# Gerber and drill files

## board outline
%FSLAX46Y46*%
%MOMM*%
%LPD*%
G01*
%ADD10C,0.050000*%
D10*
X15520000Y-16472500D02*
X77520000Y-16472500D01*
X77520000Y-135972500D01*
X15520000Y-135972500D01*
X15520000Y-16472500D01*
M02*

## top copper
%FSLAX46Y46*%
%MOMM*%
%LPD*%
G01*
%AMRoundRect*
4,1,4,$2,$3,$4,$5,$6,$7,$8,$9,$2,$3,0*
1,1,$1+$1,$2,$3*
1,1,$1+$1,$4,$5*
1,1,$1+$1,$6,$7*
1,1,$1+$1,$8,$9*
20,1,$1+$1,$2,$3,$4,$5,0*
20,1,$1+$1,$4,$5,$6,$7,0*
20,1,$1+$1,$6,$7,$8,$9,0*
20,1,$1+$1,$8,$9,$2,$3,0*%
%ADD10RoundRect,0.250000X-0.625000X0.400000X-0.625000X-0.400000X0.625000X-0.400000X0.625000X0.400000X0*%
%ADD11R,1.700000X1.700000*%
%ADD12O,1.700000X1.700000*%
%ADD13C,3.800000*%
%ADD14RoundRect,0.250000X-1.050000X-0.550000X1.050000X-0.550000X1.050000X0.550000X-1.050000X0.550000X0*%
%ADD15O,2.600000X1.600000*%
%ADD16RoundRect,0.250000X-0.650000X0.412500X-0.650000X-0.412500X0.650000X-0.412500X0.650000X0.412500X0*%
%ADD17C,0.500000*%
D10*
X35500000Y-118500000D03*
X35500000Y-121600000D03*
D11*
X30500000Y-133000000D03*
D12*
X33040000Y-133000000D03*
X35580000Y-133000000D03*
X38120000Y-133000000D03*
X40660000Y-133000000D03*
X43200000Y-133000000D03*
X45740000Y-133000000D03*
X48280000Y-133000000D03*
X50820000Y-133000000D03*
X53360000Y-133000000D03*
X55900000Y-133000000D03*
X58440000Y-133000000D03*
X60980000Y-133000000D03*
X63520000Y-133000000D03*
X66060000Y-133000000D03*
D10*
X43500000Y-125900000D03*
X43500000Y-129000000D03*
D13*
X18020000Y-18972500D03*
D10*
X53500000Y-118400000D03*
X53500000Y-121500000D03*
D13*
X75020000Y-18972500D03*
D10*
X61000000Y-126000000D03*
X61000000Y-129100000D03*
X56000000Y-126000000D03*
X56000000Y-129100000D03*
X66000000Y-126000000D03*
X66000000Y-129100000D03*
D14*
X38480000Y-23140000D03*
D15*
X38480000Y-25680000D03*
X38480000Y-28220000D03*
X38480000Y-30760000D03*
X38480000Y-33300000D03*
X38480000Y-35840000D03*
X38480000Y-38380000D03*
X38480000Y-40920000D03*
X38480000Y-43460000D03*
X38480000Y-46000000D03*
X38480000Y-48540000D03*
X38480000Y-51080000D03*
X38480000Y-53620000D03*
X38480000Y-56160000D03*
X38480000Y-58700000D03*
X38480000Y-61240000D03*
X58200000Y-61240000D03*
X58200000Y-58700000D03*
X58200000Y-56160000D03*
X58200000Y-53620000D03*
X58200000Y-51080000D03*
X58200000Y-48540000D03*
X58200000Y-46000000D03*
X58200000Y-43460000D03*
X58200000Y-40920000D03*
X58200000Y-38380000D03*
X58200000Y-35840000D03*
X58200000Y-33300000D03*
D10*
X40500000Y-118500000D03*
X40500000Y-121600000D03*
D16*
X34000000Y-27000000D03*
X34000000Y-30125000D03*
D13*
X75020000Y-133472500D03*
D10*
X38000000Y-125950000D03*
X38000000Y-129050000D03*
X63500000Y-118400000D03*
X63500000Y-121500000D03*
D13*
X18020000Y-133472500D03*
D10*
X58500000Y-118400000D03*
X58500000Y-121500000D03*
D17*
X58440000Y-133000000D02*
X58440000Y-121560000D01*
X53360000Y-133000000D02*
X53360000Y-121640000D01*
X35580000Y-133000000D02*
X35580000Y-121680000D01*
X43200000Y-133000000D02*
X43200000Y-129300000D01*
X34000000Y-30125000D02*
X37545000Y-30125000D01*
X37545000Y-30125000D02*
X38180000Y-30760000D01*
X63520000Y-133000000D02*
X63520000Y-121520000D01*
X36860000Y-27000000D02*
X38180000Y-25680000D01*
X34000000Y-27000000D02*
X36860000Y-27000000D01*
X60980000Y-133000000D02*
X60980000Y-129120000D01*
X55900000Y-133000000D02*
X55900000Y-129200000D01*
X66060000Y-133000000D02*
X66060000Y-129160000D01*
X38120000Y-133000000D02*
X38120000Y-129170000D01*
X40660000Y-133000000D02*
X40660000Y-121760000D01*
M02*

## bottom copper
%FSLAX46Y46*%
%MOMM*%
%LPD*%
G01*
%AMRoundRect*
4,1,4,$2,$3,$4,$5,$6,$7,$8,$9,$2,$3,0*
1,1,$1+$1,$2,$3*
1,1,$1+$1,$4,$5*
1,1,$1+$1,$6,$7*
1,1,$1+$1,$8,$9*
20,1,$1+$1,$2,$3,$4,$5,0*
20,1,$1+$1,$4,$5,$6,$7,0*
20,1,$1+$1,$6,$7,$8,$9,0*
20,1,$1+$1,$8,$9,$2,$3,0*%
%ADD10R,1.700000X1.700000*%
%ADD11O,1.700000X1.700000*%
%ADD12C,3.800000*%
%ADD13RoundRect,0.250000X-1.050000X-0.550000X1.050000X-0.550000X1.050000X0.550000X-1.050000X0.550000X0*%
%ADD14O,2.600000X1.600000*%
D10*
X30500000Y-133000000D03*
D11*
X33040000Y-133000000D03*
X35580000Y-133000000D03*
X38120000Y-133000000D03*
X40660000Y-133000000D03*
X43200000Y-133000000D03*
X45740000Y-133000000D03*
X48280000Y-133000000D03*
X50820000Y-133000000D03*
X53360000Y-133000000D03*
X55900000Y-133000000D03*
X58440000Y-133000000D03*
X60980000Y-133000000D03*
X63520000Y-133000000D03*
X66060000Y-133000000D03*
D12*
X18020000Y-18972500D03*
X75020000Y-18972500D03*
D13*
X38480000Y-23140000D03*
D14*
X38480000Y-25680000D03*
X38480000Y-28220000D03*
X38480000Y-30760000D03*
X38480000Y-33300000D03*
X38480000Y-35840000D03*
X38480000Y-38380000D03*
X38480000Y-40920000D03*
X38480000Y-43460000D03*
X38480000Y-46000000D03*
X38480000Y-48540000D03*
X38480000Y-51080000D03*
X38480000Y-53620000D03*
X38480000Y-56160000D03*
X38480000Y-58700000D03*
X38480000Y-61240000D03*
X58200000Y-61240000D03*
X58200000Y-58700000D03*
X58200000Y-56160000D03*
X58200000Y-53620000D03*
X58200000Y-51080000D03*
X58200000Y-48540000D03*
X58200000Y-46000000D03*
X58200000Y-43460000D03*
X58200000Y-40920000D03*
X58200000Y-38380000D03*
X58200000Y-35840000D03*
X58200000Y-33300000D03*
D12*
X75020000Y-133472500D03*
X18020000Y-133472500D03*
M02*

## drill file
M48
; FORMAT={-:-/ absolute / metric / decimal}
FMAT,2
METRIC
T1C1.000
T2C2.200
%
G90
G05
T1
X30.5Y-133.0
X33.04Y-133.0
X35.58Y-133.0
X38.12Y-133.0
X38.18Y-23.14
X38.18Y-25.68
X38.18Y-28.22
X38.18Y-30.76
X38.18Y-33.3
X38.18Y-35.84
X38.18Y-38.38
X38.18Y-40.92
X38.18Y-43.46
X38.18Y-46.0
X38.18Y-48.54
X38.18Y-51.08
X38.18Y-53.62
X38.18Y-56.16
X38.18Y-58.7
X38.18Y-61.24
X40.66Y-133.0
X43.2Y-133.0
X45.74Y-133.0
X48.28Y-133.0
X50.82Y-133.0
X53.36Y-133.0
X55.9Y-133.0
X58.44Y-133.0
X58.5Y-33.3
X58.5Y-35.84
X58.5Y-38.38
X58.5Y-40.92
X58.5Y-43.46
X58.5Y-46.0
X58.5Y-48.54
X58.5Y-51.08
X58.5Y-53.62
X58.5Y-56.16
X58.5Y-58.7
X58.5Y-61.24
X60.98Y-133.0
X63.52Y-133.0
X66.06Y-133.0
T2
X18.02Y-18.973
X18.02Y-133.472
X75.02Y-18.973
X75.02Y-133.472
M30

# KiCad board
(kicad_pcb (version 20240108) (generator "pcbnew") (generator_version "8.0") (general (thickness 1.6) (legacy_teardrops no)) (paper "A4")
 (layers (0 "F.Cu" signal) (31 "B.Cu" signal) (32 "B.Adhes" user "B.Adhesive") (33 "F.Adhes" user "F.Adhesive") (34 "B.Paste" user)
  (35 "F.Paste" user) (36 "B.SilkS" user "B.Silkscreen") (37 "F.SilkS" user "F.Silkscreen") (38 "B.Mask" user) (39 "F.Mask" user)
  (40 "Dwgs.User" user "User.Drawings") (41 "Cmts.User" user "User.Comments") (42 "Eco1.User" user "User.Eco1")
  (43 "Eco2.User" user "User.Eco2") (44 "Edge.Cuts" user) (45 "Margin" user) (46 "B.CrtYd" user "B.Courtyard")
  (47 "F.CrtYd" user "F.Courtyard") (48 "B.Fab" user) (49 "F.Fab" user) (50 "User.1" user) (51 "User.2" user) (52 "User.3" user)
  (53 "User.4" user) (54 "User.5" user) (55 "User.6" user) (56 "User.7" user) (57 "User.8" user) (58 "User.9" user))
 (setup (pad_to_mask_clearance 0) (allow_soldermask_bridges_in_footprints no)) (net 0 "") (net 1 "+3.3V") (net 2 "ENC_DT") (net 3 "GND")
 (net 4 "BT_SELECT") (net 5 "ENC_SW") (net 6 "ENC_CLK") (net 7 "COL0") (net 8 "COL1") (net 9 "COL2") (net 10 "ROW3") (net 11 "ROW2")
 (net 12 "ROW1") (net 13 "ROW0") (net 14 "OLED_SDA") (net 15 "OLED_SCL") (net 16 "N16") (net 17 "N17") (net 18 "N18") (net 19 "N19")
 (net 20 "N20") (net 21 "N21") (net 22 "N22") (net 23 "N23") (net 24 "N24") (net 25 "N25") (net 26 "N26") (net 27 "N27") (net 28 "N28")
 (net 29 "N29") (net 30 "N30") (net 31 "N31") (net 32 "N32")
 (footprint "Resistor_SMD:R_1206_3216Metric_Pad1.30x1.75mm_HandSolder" (layer "F.Cu") (at 35.5 120.05 -90)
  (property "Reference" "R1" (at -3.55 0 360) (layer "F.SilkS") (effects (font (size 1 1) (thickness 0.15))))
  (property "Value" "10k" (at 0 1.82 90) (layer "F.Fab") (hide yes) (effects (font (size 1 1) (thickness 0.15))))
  (pad "1" smd roundrect (at -1.55 0 270) (size 1.3 1.75) (layers "F.Cu" "F.Paste" "F.Mask") (roundrect_rratio 0.192308) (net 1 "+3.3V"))
  (pad "2" smd roundrect (at 1.55 0 270) (size 1.3 1.75) (layers "F.Cu" "F.Paste" "F.Mask") (roundrect_rratio 0.192308) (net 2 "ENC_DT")))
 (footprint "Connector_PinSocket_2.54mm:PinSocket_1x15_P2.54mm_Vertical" (layer "F.Cu") (at 30.5 133 90)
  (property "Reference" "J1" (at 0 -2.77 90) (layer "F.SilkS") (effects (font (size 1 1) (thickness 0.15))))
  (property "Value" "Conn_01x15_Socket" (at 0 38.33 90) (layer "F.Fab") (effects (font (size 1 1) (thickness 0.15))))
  (pad "1" thru_hole rect (at 0 0 90) (size 1.7 1.7) (drill 1) (layers "*.Cu" "*.Mask") (remove_unused_layers no) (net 1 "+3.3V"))
  (pad "2" thru_hole oval (at 0 2.54 90) (size 1.7 1.7) (drill 1) (layers "*.Cu" "*.Mask") (remove_unused_layers no) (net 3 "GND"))
  (pad "3" thru_hole oval (at 0 5.08 90) (size 1.7 1.7) (drill 1) (layers "*.Cu" "*.Mask") (remove_unused_layers no) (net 2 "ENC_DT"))
  (pad "4" thru_hole oval (at 0 7.62 90) (size 1.7 1.7) (drill 1) (layers "*.Cu" "*.Mask") (remove_unused_layers no) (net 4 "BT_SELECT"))
  (pad "5" thru_hole oval (at 0 10.16 90) (size 1.7 1.7) (drill 1) (layers "*.Cu" "*.Mask") (remove_unused_layers no) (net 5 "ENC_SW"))
  (pad "6" thru_hole oval (at 0 12.7 90) (size 1.7 1.7) (drill 1) (layers "*.Cu" "*.Mask") (remove_unused_layers no) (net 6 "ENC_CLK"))
  (pad "7" thru_hole oval (at 0 15.24 90) (size 1.7 1.7) (drill 1) (layers "*.Cu" "*.Mask") (remove_unused_layers no) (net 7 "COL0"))
  (pad "8" thru_hole oval (at 0 17.78 90) (size 1.7 1.7) (drill 1) (layers "*.Cu" "*.Mask") (remove_unused_layers no) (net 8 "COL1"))
  (pad "9" thru_hole oval (at 0 20.32 90) (size 1.7 1.7) (drill 1) (layers "*.Cu" "*.Mask") (remove_unused_layers no) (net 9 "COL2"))
  (pad "10" thru_hole oval (at 0 22.86 90) (size 1.7 1.7) (drill 1) (layers "*.Cu" "*.Mask") (remove_unused_layers no) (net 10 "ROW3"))
  (pad "11" thru_hole oval (at 0 25.4 90) (size 1.7 1.7) (drill 1) (layers "*.Cu" "*.Mask") (remove_unused_layers no) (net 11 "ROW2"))
  (pad "12" thru_hole oval (at 0 27.94 90) (size 1.7 1.7) (drill 1) (layers "*.Cu" "*.Mask") (remove_unused_layers no) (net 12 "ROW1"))
  (pad "13" thru_hole oval (at 0 30.48 90) (size 1.7 1.7) (drill 1) (layers "*.Cu" "*.Mask") (remove_unused_layers no) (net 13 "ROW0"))
  (pad "14" thru_hole oval (at 0 33.02 90) (size 1.7 1.7) (drill 1) (layers "*.Cu" "*.Mask") (remove_unused_layers no) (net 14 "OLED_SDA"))
  (pad "15" thru_hole oval (at 0 35.56 90) (size 1.7 1.7) (drill 1) (layers "*.Cu" "*.Mask") (remove_unused_layers no) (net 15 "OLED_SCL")))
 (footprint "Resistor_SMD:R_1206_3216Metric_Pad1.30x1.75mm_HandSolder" (layer "F.Cu") (at 43.5 127.45 -90)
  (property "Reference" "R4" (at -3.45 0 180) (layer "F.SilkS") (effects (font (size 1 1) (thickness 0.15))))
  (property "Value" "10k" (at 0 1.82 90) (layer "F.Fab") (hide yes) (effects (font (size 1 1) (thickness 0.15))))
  (pad "1" smd roundrect (at -1.55 0 270) (size 1.3 1.75) (layers "F.Cu" "F.Paste" "F.Mask") (roundrect_rratio 0.192308) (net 1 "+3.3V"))
  (pad "2" smd roundrect (at 1.55 0 270) (size 1.3 1.75) (layers "F.Cu" "F.Paste" "F.Mask") (roundrect_rratio 0.192308) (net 6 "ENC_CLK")))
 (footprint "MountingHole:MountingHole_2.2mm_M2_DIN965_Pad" (layer "F.Cu") (at 18.02 18.9725)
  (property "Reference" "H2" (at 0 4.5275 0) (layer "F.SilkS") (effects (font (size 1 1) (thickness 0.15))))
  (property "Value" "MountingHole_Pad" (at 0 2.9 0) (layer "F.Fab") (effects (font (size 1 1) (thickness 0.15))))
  (pad "1" thru_hole circle (at 0 0) (size 3.8 3.8) (drill 2.2) (layers "*.Cu" "*.Mask") (remove_unused_layers no) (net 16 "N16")))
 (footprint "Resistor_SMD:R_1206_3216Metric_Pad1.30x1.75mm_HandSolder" (layer "F.Cu") (at 53.5 119.95 -90)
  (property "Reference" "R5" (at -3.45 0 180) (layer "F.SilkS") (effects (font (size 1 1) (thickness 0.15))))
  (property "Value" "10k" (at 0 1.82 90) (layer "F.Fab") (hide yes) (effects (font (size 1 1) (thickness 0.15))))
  (pad "1" smd roundrect (at -1.55 0 270) (size 1.3 1.75) (layers "F.Cu" "F.Paste" "F.Mask") (roundrect_rratio 0.192308) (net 1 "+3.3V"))
  (pad "2" smd roundrect (at 1.55 0 270) (size 1.3 1.75) (layers "F.Cu" "F.Paste" "F.Mask") (roundrect_rratio 0.192308) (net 10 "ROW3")))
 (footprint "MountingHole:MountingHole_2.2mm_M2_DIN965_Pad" (layer "F.Cu") (at 75.02 18.9725)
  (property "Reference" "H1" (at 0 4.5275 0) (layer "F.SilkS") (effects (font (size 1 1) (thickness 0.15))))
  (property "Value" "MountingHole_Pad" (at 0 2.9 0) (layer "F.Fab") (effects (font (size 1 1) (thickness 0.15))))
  (pad "1" thru_hole circle (at 0 0) (size 3.8 3.8) (drill 2.2) (layers "*.Cu" "*.Mask") (remove_unused_layers no) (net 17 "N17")))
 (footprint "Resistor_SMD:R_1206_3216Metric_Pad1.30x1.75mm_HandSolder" (layer "F.Cu") (at 61 127.55 -90)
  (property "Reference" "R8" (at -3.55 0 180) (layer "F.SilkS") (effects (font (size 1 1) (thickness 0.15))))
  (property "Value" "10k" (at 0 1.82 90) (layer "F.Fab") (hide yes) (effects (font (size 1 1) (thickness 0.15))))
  (pad "1" smd roundrect (at -1.55 0 270) (size 1.3 1.75) (layers "F.Cu" "F.Paste" "F.Mask") (roundrect_rratio 0.192308) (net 1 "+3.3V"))
  (pad "2" smd roundrect (at 1.55 0 270) (size 1.3 1.75) (layers "F.Cu" "F.Paste" "F.Mask") (roundrect_rratio 0.192308) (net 13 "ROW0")))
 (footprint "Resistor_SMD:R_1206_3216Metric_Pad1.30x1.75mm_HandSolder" (layer "F.Cu") (at 56 127.55 -90)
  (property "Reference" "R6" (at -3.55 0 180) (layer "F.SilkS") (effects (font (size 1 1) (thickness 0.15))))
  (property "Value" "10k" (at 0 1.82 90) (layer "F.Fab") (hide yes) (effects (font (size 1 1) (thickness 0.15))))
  (pad "1" smd roundrect (at -1.55 0 270) (size 1.3 1.75) (layers "F.Cu" "F.Paste" "F.Mask") (roundrect_rratio 0.192308) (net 1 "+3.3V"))
  (pad "2" smd roundrect (at 1.55 0 270) (size 1.3 1.75) (layers "F.Cu" "F.Paste" "F.Mask") (roundrect_rratio 0.192308) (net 11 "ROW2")))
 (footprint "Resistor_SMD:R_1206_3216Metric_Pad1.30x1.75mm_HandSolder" (layer "F.Cu") (at 66 127.55 -90)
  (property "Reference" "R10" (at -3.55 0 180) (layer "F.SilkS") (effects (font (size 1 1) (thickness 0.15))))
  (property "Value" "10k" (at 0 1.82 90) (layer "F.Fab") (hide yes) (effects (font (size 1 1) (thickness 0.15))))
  (pad "1" smd roundrect (at -1.55 0 270) (size 1.3 1.75) (layers "F.Cu" "F.Paste" "F.Mask") (roundrect_rratio 0.192308) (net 1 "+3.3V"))
  (pad "2" smd roundrect (at 1.55 0 270) (size 1.3 1.75) (layers "F.Cu" "F.Paste" "F.Mask") (roundrect_rratio 0.192308) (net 15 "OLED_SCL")))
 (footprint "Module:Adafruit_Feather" (layer "F.Cu") (at 38.18 23.14)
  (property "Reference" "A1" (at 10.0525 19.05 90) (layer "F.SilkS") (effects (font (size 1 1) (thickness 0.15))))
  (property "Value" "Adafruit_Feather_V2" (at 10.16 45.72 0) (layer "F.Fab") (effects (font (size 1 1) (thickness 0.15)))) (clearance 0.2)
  (pad "1" thru_hole roundrect (at 0 0) (size 2.6 1.6) (drill 1 (offset 0.3 0)) (layers "*.Cu" "*.Mask") (remove_unused_layers no)
   (roundrect_rratio 0.15625) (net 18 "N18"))
  (pad "2" thru_hole oval (at 0 2.54) (size 2.6 1.6) (drill 1 (offset 0.3 0)) (layers "*.Cu" "*.Mask") (remove_unused_layers no)
   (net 1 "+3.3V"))
  (pad "3" thru_hole oval (at 0 5.08) (size 2.6 1.6) (drill 1 (offset 0.3 0)) (layers "*.Cu" "*.Mask") (remove_unused_layers no)
   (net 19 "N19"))
  (pad "4" thru_hole oval (at 0 7.62) (size 2.6 1.6) (drill 1 (offset 0.3 0)) (layers "*.Cu" "*.Mask") (remove_unused_layers no)
   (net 3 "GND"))
  (pad "5" thru_hole oval (at 0 10.16) (size 2.6 1.6) (drill 1 (offset 0.3 0)) (layers "*.Cu" "*.Mask") (remove_unused_layers no)
   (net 2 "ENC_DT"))
  (pad "6" thru_hole oval (at 0 12.7) (size 2.6 1.6) (drill 1 (offset 0.3 0)) (layers "*.Cu" "*.Mask") (remove_unused_layers no)
   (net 4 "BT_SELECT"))
  (pad "7" thru_hole oval (at 0 15.24) (size 2.6 1.6) (drill 1 (offset 0.3 0)) (layers "*.Cu" "*.Mask") (remove_unused_layers no)
   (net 5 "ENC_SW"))
  (pad "8" thru_hole oval (at 0 17.78) (size 2.6 1.6) (drill 1 (offset 0.3 0)) (layers "*.Cu" "*.Mask") (remove_unused_layers no)
   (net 6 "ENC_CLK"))
  (pad "9" thru_hole oval (at 0 20.32) (size 2.6 1.6) (drill 1 (offset 0.3 0)) (layers "*.Cu" "*.Mask") (remove_unused_layers no)
   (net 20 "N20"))
  (pad "10" thru_hole oval (at 0 22.86) (size 2.6 1.6) (drill 1 (offset 0.3 0)) (layers "*.Cu" "*.Mask") (remove_unused_layers no)
   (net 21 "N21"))
  (pad "11" thru_hole oval (at 0 25.4) (size 2.6 1.6) (drill 1 (offset 0.3 0)) (layers "*.Cu" "*.Mask") (remove_unused_layers no)
   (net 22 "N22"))
  (pad "12" thru_hole oval (at 0 27.94) (size 2.6 1.6) (drill 1 (offset 0.3 0)) (layers "*.Cu" "*.Mask") (remove_unused_layers no)
   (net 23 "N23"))
  (pad "13" thru_hole oval (at 0 30.48) (size 2.6 1.6) (drill 1 (offset 0.3 0)) (layers "*.Cu" "*.Mask") (remove_unused_layers no)
   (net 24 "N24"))
  (pad "14" thru_hole oval (at 0 33.02) (size 2.6 1.6) (drill 1 (offset 0.3 0)) (layers "*.Cu" "*.Mask") (remove_unused_layers no)
   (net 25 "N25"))
  (pad "15" thru_hole oval (at 0 35.56) (size 2.6 1.6) (drill 1 (offset 0.3 0)) (layers "*.Cu" "*.Mask") (remove_unused_layers no)
   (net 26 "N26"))
  (pad "16" thru_hole oval (at 0 38.1) (size 2.6 1.6) (drill 1 (offset 0.3 0)) (layers "*.Cu" "*.Mask") (remove_unused_layers no)
   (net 13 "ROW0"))
  (pad "17" thru_hole oval (at 20.32 38.1 180) (size 2.6 1.6) (drill 1 (offset 0.3 0)) (layers "*.Cu" "*.Mask") (remove_unused_layers no)
   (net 14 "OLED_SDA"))
  (pad "18" thru_hole oval (at 20.32 35.56 180) (size 2.6 1.6) (drill 1 (offset 0.3 0)) (layers "*.Cu" "*.Mask") (remove_unused_layers no)
   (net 15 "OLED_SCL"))
  (pad "19" thru_hole oval (at 20.32 33.02 180) (size 2.6 1.6) (drill 1 (offset 0.3 0)) (layers "*.Cu" "*.Mask") (remove_unused_layers no)
   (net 12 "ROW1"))
  (pad "20" thru_hole oval (at 20.32 30.48 180) (size 2.6 1.6) (drill 1 (offset 0.3 0)) (layers "*.Cu" "*.Mask") (remove_unused_layers no)
   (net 11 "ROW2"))
  (pad "21" thru_hole oval (at 20.32 27.94 180) (size 2.6 1.6) (drill 1 (offset 0.3 0)) (layers "*.Cu" "*.Mask") (remove_unused_layers no)
   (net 10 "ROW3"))
  (pad "22" thru_hole oval (at 20.32 25.4 180) (size 2.6 1.6) (drill 1 (offset 0.3 0)) (layers "*.Cu" "*.Mask") (remove_unused_layers no)
   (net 9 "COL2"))
  (pad "23" thru_hole oval (at 20.32 22.86 180) (size 2.6 1.6) (drill 1 (offset 0.3 0)) (layers "*.Cu" "*.Mask") (remove_unused_layers no)
   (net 8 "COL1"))
  (pad "24" thru_hole oval (at 20.32 20.32 180) (size 2.6 1.6) (drill 1 (offset 0.3 0)) (layers "*.Cu" "*.Mask") (remove_unused_layers no)
   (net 7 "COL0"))
  (pad "25" thru_hole oval (at 20.32 17.78 180) (size 2.6 1.6) (drill 1 (offset 0.3 0)) (layers "*.Cu" "*.Mask") (remove_unused_layers no)
   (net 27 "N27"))
  (pad "26" thru_hole oval (at 20.32 15.24 180) (size 2.6 1.6) (drill 1 (offset 0.3 0)) (layers "*.Cu" "*.Mask") (remove_unused_layers no)
   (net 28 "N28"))
  (pad "27" thru_hole oval (at 20.32 12.7 180) (size 2.6 1.6) (drill 1 (offset 0.3 0)) (layers "*.Cu" "*.Mask") (remove_unused_layers no)
   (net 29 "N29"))
  (pad "28" thru_hole oval (at 20.32 10.16 180) (size 2.6 1.6) (drill 1 (offset 0.3 0)) (layers "*.Cu" "*.Mask") (remove_unused_layers no)
   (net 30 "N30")))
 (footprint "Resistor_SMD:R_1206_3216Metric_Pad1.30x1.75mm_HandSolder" (layer "F.Cu") (at 40.5 120.05 -90)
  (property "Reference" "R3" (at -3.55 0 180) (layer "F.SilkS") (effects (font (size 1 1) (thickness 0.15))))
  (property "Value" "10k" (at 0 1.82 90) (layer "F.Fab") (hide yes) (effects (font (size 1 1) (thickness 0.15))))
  (pad "1" smd roundrect (at -1.55 0 270) (size 1.3 1.75) (layers "F.Cu" "F.Paste" "F.Mask") (roundrect_rratio 0.192308) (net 1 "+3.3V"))
  (pad "2" smd roundrect (at 1.55 0 270) (size 1.3 1.75) (layers "F.Cu" "F.Paste" "F.Mask") (roundrect_rratio 0.192308) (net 5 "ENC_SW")))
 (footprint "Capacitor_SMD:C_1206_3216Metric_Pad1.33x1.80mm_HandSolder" (layer "F.Cu") (at 34 28.5625 -90)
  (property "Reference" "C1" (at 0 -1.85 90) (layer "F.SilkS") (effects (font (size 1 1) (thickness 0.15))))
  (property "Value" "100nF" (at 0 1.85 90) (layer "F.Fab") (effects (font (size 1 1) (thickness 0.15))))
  (pad "1" smd roundrect (at -1.5625 0 270) (size 1.325 1.8) (layers "F.Cu" "F.Paste" "F.Mask") (roundrect_rratio 0.188679) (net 1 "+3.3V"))
  (pad "2" smd roundrect (at 1.5625 0 270) (size 1.325 1.8) (layers "F.Cu" "F.Paste" "F.Mask") (roundrect_rratio 0.188679) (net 3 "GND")))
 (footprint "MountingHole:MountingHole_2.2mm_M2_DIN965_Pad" (layer "F.Cu") (at 75.02 133.4725)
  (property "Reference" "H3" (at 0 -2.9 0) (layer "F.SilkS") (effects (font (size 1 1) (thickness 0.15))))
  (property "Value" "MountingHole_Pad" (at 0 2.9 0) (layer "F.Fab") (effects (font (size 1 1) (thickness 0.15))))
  (pad "1" thru_hole circle (at 0 0) (size 3.8 3.8) (drill 2.2) (layers "*.Cu" "*.Mask") (remove_unused_layers no) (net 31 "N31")))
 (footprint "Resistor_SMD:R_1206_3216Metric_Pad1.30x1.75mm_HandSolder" (layer "F.Cu") (at 38 127.5 -90)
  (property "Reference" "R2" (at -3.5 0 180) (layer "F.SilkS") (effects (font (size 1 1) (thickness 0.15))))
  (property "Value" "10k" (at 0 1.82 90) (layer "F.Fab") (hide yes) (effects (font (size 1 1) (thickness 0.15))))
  (pad "1" smd roundrect (at -1.55 0 270) (size 1.3 1.75) (layers "F.Cu" "F.Paste" "F.Mask") (roundrect_rratio 0.192308) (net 1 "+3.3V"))
  (pad "2" smd roundrect (at 1.55 0 270) (size 1.3 1.75) (layers "F.Cu" "F.Paste" "F.Mask") (roundrect_rratio 0.192308) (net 4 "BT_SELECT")))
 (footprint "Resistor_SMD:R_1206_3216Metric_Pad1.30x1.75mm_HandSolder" (layer "F.Cu") (at 63.5 119.95 -90)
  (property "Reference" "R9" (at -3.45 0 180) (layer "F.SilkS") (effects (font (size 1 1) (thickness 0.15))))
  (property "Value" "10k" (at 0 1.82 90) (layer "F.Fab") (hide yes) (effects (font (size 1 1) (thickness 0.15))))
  (pad "1" smd roundrect (at -1.55 0 270) (size 1.3 1.75) (layers "F.Cu" "F.Paste" "F.Mask") (roundrect_rratio 0.192308) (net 1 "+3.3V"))
  (pad "2" smd roundrect (at 1.55 0 270) (size 1.3 1.75) (layers "F.Cu" "F.Paste" "F.Mask") (roundrect_rratio 0.192308) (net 14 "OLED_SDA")))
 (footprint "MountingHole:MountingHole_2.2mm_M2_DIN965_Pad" (layer "F.Cu") (at 18.02 133.4725)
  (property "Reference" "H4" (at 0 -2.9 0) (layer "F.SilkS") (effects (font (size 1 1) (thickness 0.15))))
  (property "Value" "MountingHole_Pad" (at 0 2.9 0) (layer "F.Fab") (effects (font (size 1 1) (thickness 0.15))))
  (pad "1" thru_hole circle (at 0 0) (size 3.8 3.8) (drill 2.2) (layers "*.Cu" "*.Mask") (remove_unused_layers no) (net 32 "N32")))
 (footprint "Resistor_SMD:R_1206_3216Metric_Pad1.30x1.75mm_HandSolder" (layer "F.Cu") (at 58.5 119.95 -90)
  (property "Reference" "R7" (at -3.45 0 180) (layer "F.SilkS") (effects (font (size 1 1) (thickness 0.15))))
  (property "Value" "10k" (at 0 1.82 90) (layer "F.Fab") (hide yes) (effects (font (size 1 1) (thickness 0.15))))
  (pad "1" smd roundrect (at -1.55 0 270) (size 1.3 1.75) (layers "F.Cu" "F.Paste" "F.Mask") (roundrect_rratio 0.192308) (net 1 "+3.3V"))
  (pad "2" smd roundrect (at 1.55 0 270) (size 1.3 1.75) (layers "F.Cu" "F.Paste" "F.Mask") (roundrect_rratio 0.192308) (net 12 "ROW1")))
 (gr_rect (start 15.52 16.4725) (end 77.52 135.9725) (stroke (width 0.05) (type default)) (fill none) (layer "Edge.Cuts"))
 (segment (start 58.44 133) (end 58.44 121.56) (width 0.5) (layer "F.Cu") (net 12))
 (segment (start 53.36 133) (end 53.36 121.64) (width 0.5) (layer "F.Cu") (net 10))
 (segment (start 35.58 133) (end 35.58 121.68) (width 0.5) (layer "F.Cu") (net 2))
 (segment (start 43.2 133) (end 43.2 129.3) (width 0.5) (layer "F.Cu") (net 6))
 (segment (start 34 30.125) (end 37.545 30.125) (width 0.5) (layer "F.Cu") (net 3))
 (segment (start 37.545 30.125) (end 38.18 30.76) (width 0.5) (layer "F.Cu") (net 3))
 (segment (start 63.52 133) (end 63.52 121.52) (width 0.5) (layer "F.Cu") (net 14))
 (segment (start 36.86 27) (end 38.18 25.68) (width 0.5) (layer "F.Cu") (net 1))
 (segment (start 34 27) (end 36.86 27) (width 0.5) (layer "F.Cu") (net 1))
 (segment (start 60.98 133) (end 60.98 129.12) (width 0.5) (layer "F.Cu") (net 13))
 (segment (start 55.9 133) (end 55.9 129.2) (width 0.5) (layer "F.Cu") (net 11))
 (segment (start 66.06 133) (end 66.06 129.16) (width 0.5) (layer "F.Cu") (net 15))
 (segment (start 38.12 133) (end 38.12 129.17) (width 0.5) (layer "F.Cu") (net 4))
 (segment (start 40.66 133) (end 40.66 121.76) (width 0.5) (layer "F.Cu") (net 5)))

